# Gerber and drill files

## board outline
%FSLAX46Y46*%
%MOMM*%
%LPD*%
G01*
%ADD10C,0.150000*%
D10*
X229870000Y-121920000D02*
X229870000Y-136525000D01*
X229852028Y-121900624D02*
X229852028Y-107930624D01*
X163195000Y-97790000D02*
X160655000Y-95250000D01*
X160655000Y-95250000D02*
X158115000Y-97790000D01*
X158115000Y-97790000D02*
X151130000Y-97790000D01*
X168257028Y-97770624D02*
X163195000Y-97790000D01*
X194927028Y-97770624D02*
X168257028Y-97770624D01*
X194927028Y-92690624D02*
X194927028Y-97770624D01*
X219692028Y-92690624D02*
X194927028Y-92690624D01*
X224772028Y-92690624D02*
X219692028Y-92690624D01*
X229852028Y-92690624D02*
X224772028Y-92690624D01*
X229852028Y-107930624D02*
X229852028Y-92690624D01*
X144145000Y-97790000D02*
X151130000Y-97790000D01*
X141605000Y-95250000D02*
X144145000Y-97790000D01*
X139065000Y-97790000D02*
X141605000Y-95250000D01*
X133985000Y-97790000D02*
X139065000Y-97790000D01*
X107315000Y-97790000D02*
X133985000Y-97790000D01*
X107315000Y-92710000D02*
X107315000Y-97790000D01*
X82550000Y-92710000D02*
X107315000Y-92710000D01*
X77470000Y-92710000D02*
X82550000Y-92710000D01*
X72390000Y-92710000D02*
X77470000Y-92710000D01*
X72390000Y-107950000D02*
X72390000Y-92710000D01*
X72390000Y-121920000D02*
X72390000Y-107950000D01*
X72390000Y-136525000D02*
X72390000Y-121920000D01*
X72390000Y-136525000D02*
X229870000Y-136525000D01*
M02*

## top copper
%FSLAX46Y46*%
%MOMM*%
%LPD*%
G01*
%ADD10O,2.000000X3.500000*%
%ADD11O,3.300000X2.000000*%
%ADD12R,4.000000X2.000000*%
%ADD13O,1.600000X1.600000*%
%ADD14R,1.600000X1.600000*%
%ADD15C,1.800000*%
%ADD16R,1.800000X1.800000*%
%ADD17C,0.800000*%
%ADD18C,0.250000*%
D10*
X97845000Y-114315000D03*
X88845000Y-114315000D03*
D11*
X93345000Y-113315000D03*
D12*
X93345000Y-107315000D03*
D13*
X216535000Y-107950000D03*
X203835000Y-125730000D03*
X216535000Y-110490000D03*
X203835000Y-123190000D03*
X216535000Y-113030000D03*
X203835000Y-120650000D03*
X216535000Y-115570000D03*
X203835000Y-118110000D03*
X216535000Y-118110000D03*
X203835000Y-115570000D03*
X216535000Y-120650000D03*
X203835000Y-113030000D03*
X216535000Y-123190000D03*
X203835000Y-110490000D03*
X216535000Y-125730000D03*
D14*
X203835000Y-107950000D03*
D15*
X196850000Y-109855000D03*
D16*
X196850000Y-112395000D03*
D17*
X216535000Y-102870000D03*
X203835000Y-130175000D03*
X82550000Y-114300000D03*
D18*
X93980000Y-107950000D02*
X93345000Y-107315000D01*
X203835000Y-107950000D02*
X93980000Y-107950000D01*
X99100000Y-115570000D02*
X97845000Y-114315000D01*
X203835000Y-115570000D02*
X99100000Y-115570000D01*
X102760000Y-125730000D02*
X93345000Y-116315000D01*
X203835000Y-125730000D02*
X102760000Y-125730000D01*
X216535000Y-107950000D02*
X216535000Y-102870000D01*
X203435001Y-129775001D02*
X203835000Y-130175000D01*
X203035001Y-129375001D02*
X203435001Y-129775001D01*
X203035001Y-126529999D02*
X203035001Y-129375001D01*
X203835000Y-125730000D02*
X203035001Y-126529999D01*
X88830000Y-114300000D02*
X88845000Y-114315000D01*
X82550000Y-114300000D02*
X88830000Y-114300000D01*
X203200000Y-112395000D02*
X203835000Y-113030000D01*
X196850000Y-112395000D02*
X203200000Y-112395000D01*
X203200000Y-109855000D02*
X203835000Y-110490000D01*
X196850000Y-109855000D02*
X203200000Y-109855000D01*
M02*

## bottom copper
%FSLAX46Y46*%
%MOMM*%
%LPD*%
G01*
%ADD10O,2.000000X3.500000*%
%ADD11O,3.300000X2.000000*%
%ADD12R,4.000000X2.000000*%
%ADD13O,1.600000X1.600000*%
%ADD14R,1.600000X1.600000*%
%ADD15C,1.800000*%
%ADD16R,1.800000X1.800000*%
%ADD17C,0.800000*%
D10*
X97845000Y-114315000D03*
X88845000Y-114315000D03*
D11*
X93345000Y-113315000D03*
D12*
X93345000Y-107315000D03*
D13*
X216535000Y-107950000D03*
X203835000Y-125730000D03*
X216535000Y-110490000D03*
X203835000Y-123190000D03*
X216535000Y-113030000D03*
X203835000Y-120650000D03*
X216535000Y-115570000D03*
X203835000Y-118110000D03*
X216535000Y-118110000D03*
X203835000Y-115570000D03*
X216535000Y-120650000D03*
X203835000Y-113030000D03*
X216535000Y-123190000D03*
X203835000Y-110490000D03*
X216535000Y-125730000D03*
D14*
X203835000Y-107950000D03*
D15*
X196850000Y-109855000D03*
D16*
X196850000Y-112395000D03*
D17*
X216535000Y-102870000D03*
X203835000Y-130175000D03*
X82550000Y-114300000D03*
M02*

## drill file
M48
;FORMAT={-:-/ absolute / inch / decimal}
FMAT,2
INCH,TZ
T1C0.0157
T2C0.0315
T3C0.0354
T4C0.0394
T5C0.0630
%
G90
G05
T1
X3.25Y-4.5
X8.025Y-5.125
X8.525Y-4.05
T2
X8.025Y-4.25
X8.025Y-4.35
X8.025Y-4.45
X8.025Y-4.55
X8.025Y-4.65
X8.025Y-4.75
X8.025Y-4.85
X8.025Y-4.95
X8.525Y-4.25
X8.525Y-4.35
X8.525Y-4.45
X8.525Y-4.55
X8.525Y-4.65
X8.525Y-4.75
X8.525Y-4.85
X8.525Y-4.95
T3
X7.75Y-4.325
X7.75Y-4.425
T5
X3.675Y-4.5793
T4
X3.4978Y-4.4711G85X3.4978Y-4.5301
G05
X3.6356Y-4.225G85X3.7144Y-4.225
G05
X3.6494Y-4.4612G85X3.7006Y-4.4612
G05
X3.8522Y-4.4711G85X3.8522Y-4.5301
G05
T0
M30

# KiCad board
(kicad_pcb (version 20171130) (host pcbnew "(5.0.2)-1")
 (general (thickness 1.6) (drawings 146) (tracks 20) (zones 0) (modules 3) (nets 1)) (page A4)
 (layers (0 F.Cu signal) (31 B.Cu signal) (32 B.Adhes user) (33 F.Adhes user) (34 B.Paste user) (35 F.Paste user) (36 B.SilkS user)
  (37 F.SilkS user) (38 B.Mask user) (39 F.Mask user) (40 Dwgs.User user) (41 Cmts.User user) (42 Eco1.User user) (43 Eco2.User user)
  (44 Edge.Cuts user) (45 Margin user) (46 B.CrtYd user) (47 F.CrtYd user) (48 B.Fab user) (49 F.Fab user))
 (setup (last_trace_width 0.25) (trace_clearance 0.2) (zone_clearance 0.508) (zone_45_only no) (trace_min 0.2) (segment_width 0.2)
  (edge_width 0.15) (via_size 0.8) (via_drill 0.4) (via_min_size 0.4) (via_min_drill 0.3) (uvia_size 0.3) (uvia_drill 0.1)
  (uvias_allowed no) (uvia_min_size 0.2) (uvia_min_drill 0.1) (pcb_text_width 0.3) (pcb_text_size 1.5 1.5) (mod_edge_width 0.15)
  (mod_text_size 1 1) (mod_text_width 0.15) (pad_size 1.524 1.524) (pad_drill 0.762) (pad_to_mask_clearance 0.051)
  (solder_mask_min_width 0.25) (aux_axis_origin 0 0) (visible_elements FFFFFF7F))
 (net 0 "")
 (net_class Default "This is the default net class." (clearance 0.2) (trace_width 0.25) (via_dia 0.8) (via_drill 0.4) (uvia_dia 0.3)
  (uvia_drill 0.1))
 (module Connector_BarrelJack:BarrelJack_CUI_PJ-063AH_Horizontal (layer F.Cu) (at 93.345 107.315)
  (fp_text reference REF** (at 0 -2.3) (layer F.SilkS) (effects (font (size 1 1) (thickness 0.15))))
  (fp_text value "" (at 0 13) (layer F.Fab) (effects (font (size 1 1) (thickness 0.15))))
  (pad "" np_thru_hole circle (at 0 9) (size 1.6 1.6) (drill 1.6) (layers *.Cu *.Mask))
  (pad MP thru_hole oval (at 4.5 7) (size 2 3.5) (drill oval 1 2.5) (layers *.Cu *.Mask))
  (pad MP thru_hole oval (at -4.5 7) (size 2 3.5) (drill oval 1 2.5) (layers *.Cu *.Mask))
  (pad 2 thru_hole oval (at 0 6) (size 3.3 2) (drill oval 2.3 1) (layers *.Cu *.Mask))
  (pad 1 thru_hole rect (at 0 0) (size 4 2) (drill oval 3 1) (layers *.Cu *.Mask)))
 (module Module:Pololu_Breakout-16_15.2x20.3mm (layer F.Cu) (at 203.835 107.95)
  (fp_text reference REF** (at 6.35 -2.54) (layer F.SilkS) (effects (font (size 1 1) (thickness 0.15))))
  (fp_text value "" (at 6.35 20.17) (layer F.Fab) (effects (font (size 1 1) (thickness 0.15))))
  (pad 16 thru_hole oval (at 12.7 0) (size 1.6 1.6) (drill 0.8) (layers *.Cu *.Mask))
  (pad 8 thru_hole oval (at 0 17.78) (size 1.6 1.6) (drill 0.8) (layers *.Cu *.Mask))
  (pad 15 thru_hole oval (at 12.7 2.54) (size 1.6 1.6) (drill 0.8) (layers *.Cu *.Mask))
  (pad 7 thru_hole oval (at 0 15.24) (size 1.6 1.6) (drill 0.8) (layers *.Cu *.Mask))
  (pad 14 thru_hole oval (at 12.7 5.08) (size 1.6 1.6) (drill 0.8) (layers *.Cu *.Mask))
  (pad 6 thru_hole oval (at 0 12.7) (size 1.6 1.6) (drill 0.8) (layers *.Cu *.Mask))
  (pad 13 thru_hole oval (at 12.7 7.62) (size 1.6 1.6) (drill 0.8) (layers *.Cu *.Mask))
  (pad 5 thru_hole oval (at 0 10.16) (size 1.6 1.6) (drill 0.8) (layers *.Cu *.Mask))
  (pad 12 thru_hole oval (at 12.7 10.16) (size 1.6 1.6) (drill 0.8) (layers *.Cu *.Mask))
  (pad 4 thru_hole oval (at 0 7.62) (size 1.6 1.6) (drill 0.8) (layers *.Cu *.Mask))
  (pad 11 thru_hole oval (at 12.7 12.7) (size 1.6 1.6) (drill 0.8) (layers *.Cu *.Mask))
  (pad 3 thru_hole oval (at 0 5.08) (size 1.6 1.6) (drill 0.8) (layers *.Cu *.Mask))
  (pad 10 thru_hole oval (at 12.7 15.24) (size 1.6 1.6) (drill 0.8) (layers *.Cu *.Mask))
  (pad 2 thru_hole oval (at 0 2.54) (size 1.6 1.6) (drill 0.8) (layers *.Cu *.Mask))
  (pad 9 thru_hole oval (at 12.7 17.78) (size 1.6 1.6) (drill 0.8) (layers *.Cu *.Mask))
  (pad 1 thru_hole rect (at 0 0) (size 1.6 1.6) (drill 0.8) (layers *.Cu *.Mask)))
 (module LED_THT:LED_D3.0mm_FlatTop (layer F.Cu) (at 196.85 112.395 90)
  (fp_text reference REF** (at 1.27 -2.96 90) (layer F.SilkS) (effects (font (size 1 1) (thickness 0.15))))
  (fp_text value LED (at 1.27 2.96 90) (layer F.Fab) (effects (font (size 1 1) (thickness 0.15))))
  (pad 2 thru_hole circle (at 2.54 0 90) (size 1.8 1.8) (drill 0.9) (layers *.Cu *.Mask))
  (pad 1 thru_hole rect (at 0 0 90) (size 1.8 1.8) (drill 0.9) (layers *.Cu *.Mask)))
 (gr_line (start 229.87 121.92) (end 229.87 136.525) (layer Edge.Cuts) (width 0.15))
 (gr_line (start 229.852028 121.900624) (end 229.852028 107.930624) (layer Edge.Cuts) (width 0.15))
 (gr_line (start 163.195 97.79) (end 160.655 95.25) (layer Edge.Cuts) (width 0.15))
 (gr_line (start 160.655 95.25) (end 158.115 97.79) (layer Edge.Cuts) (width 0.15))
 (gr_line (start 158.115 97.79) (end 151.13 97.79) (layer Edge.Cuts) (width 0.15))
 (gr_line (start 168.257028 97.770624) (end 163.195 97.79) (layer Edge.Cuts) (width 0.15))
 (gr_line (start 194.927028 97.770624) (end 168.257028 97.770624) (layer Edge.Cuts) (width 0.15))
 (gr_line (start 194.927028 92.690624) (end 194.927028 97.770624) (layer Edge.Cuts) (width 0.15))
 (gr_line (start 219.692028 92.690624) (end 194.927028 92.690624) (layer Edge.Cuts) (width 0.15))
 (gr_line (start 224.772028 92.690624) (end 219.692028 92.690624) (layer Edge.Cuts) (width 0.15))
 (gr_line (start 229.852028 92.690624) (end 224.772028 92.690624) (layer Edge.Cuts) (width 0.15))
 (gr_line (start 229.852028 107.930624) (end 229.852028 92.690624) (layer Edge.Cuts) (width 0.15))
 (gr_line (start 144.145 97.79) (end 151.13 97.79) (layer Edge.Cuts) (width 0.15))
 (gr_line (start 141.605 95.25) (end 144.145 97.79) (layer Edge.Cuts) (width 0.15))
 (gr_line (start 139.065 97.79) (end 141.605 95.25) (layer Edge.Cuts) (width 0.15))
 (gr_line (start 133.985 97.79) (end 139.065 97.79) (layer Edge.Cuts) (width 0.15))
 (gr_line (start 107.315 97.79) (end 133.985 97.79) (layer Edge.Cuts) (width 0.15))
 (gr_line (start 107.315 92.71) (end 107.315 97.79) (layer Edge.Cuts) (width 0.15))
 (gr_line (start 82.55 92.71) (end 107.315 92.71) (layer Edge.Cuts) (width 0.15))
 (gr_line (start 77.47 92.71) (end 82.55 92.71) (layer Edge.Cuts) (width 0.15))
 (gr_line (start 72.39 92.71) (end 77.47 92.71) (layer Edge.Cuts) (width 0.15))
 (gr_line (start 72.39 107.95) (end 72.39 92.71) (layer Edge.Cuts) (width 0.15))
 (gr_line (start 72.39 121.92) (end 72.39 107.95) (layer Edge.Cuts) (width 0.15))
 (gr_line (start 72.39 136.525) (end 72.39 121.92) (layer Edge.Cuts) (width 0.15))
 (gr_line (start 72.39 136.525) (end 229.87 136.525) (layer Edge.Cuts) (width 0.15))
 (segment (start 93.98 107.95) (end 93.345 107.315) (width 0.25) (layer F.Cu) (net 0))
 (segment (start 203.835 107.95) (end 93.98 107.95) (width 0.25) (layer F.Cu) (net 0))
 (segment (start 99.1 115.57) (end 97.845 114.315) (width 0.25) (layer F.Cu) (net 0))
 (segment (start 203.835 115.57) (end 99.1 115.57) (width 0.25) (layer F.Cu) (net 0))
 (segment (start 102.76 125.73) (end 93.345 116.315) (width 0.25) (layer F.Cu) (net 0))
 (segment (start 203.835 125.73) (end 102.76 125.73) (width 0.25) (layer F.Cu) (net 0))
 (via (at 216.535 102.87) (size 0.8) (drill 0.4) (layers F.Cu B.Cu) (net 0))
 (segment (start 216.535 107.95) (end 216.535 102.87) (width 0.25) (layer F.Cu) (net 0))
 (via (at 203.835 130.175) (size 0.8) (drill 0.4) (layers F.Cu B.Cu) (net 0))
 (segment (start 203.435001 129.775001) (end 203.835 130.175) (width 0.25) (layer F.Cu) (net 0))
 (segment (start 203.035001 129.375001) (end 203.435001 129.775001) (width 0.25) (layer F.Cu) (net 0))
 (segment (start 203.035001 126.529999) (end 203.035001 129.375001) (width 0.25) (layer F.Cu) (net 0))
 (segment (start 203.835 125.73) (end 203.035001 126.529999) (width 0.25) (layer F.Cu) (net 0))
 (via (at 82.55 114.3) (size 0.8) (drill 0.4) (layers F.Cu B.Cu) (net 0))
 (segment (start 88.83 114.3) (end 88.845 114.315) (width 0.25) (layer F.Cu) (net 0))
 (segment (start 82.55 114.3) (end 88.83 114.3) (width 0.25) (layer F.Cu) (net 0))
 (segment (start 203.2 112.395) (end 203.835 113.03) (width 0.25) (layer F.Cu) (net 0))
 (segment (start 196.85 112.395) (end 203.2 112.395) (width 0.25) (layer F.Cu) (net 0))
 (segment (start 203.2 109.855) (end 203.835 110.49) (width 0.25) (layer F.Cu) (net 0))
 (segment (start 196.85 109.855) (end 203.2 109.855) (width 0.25) (layer F.Cu) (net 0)))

